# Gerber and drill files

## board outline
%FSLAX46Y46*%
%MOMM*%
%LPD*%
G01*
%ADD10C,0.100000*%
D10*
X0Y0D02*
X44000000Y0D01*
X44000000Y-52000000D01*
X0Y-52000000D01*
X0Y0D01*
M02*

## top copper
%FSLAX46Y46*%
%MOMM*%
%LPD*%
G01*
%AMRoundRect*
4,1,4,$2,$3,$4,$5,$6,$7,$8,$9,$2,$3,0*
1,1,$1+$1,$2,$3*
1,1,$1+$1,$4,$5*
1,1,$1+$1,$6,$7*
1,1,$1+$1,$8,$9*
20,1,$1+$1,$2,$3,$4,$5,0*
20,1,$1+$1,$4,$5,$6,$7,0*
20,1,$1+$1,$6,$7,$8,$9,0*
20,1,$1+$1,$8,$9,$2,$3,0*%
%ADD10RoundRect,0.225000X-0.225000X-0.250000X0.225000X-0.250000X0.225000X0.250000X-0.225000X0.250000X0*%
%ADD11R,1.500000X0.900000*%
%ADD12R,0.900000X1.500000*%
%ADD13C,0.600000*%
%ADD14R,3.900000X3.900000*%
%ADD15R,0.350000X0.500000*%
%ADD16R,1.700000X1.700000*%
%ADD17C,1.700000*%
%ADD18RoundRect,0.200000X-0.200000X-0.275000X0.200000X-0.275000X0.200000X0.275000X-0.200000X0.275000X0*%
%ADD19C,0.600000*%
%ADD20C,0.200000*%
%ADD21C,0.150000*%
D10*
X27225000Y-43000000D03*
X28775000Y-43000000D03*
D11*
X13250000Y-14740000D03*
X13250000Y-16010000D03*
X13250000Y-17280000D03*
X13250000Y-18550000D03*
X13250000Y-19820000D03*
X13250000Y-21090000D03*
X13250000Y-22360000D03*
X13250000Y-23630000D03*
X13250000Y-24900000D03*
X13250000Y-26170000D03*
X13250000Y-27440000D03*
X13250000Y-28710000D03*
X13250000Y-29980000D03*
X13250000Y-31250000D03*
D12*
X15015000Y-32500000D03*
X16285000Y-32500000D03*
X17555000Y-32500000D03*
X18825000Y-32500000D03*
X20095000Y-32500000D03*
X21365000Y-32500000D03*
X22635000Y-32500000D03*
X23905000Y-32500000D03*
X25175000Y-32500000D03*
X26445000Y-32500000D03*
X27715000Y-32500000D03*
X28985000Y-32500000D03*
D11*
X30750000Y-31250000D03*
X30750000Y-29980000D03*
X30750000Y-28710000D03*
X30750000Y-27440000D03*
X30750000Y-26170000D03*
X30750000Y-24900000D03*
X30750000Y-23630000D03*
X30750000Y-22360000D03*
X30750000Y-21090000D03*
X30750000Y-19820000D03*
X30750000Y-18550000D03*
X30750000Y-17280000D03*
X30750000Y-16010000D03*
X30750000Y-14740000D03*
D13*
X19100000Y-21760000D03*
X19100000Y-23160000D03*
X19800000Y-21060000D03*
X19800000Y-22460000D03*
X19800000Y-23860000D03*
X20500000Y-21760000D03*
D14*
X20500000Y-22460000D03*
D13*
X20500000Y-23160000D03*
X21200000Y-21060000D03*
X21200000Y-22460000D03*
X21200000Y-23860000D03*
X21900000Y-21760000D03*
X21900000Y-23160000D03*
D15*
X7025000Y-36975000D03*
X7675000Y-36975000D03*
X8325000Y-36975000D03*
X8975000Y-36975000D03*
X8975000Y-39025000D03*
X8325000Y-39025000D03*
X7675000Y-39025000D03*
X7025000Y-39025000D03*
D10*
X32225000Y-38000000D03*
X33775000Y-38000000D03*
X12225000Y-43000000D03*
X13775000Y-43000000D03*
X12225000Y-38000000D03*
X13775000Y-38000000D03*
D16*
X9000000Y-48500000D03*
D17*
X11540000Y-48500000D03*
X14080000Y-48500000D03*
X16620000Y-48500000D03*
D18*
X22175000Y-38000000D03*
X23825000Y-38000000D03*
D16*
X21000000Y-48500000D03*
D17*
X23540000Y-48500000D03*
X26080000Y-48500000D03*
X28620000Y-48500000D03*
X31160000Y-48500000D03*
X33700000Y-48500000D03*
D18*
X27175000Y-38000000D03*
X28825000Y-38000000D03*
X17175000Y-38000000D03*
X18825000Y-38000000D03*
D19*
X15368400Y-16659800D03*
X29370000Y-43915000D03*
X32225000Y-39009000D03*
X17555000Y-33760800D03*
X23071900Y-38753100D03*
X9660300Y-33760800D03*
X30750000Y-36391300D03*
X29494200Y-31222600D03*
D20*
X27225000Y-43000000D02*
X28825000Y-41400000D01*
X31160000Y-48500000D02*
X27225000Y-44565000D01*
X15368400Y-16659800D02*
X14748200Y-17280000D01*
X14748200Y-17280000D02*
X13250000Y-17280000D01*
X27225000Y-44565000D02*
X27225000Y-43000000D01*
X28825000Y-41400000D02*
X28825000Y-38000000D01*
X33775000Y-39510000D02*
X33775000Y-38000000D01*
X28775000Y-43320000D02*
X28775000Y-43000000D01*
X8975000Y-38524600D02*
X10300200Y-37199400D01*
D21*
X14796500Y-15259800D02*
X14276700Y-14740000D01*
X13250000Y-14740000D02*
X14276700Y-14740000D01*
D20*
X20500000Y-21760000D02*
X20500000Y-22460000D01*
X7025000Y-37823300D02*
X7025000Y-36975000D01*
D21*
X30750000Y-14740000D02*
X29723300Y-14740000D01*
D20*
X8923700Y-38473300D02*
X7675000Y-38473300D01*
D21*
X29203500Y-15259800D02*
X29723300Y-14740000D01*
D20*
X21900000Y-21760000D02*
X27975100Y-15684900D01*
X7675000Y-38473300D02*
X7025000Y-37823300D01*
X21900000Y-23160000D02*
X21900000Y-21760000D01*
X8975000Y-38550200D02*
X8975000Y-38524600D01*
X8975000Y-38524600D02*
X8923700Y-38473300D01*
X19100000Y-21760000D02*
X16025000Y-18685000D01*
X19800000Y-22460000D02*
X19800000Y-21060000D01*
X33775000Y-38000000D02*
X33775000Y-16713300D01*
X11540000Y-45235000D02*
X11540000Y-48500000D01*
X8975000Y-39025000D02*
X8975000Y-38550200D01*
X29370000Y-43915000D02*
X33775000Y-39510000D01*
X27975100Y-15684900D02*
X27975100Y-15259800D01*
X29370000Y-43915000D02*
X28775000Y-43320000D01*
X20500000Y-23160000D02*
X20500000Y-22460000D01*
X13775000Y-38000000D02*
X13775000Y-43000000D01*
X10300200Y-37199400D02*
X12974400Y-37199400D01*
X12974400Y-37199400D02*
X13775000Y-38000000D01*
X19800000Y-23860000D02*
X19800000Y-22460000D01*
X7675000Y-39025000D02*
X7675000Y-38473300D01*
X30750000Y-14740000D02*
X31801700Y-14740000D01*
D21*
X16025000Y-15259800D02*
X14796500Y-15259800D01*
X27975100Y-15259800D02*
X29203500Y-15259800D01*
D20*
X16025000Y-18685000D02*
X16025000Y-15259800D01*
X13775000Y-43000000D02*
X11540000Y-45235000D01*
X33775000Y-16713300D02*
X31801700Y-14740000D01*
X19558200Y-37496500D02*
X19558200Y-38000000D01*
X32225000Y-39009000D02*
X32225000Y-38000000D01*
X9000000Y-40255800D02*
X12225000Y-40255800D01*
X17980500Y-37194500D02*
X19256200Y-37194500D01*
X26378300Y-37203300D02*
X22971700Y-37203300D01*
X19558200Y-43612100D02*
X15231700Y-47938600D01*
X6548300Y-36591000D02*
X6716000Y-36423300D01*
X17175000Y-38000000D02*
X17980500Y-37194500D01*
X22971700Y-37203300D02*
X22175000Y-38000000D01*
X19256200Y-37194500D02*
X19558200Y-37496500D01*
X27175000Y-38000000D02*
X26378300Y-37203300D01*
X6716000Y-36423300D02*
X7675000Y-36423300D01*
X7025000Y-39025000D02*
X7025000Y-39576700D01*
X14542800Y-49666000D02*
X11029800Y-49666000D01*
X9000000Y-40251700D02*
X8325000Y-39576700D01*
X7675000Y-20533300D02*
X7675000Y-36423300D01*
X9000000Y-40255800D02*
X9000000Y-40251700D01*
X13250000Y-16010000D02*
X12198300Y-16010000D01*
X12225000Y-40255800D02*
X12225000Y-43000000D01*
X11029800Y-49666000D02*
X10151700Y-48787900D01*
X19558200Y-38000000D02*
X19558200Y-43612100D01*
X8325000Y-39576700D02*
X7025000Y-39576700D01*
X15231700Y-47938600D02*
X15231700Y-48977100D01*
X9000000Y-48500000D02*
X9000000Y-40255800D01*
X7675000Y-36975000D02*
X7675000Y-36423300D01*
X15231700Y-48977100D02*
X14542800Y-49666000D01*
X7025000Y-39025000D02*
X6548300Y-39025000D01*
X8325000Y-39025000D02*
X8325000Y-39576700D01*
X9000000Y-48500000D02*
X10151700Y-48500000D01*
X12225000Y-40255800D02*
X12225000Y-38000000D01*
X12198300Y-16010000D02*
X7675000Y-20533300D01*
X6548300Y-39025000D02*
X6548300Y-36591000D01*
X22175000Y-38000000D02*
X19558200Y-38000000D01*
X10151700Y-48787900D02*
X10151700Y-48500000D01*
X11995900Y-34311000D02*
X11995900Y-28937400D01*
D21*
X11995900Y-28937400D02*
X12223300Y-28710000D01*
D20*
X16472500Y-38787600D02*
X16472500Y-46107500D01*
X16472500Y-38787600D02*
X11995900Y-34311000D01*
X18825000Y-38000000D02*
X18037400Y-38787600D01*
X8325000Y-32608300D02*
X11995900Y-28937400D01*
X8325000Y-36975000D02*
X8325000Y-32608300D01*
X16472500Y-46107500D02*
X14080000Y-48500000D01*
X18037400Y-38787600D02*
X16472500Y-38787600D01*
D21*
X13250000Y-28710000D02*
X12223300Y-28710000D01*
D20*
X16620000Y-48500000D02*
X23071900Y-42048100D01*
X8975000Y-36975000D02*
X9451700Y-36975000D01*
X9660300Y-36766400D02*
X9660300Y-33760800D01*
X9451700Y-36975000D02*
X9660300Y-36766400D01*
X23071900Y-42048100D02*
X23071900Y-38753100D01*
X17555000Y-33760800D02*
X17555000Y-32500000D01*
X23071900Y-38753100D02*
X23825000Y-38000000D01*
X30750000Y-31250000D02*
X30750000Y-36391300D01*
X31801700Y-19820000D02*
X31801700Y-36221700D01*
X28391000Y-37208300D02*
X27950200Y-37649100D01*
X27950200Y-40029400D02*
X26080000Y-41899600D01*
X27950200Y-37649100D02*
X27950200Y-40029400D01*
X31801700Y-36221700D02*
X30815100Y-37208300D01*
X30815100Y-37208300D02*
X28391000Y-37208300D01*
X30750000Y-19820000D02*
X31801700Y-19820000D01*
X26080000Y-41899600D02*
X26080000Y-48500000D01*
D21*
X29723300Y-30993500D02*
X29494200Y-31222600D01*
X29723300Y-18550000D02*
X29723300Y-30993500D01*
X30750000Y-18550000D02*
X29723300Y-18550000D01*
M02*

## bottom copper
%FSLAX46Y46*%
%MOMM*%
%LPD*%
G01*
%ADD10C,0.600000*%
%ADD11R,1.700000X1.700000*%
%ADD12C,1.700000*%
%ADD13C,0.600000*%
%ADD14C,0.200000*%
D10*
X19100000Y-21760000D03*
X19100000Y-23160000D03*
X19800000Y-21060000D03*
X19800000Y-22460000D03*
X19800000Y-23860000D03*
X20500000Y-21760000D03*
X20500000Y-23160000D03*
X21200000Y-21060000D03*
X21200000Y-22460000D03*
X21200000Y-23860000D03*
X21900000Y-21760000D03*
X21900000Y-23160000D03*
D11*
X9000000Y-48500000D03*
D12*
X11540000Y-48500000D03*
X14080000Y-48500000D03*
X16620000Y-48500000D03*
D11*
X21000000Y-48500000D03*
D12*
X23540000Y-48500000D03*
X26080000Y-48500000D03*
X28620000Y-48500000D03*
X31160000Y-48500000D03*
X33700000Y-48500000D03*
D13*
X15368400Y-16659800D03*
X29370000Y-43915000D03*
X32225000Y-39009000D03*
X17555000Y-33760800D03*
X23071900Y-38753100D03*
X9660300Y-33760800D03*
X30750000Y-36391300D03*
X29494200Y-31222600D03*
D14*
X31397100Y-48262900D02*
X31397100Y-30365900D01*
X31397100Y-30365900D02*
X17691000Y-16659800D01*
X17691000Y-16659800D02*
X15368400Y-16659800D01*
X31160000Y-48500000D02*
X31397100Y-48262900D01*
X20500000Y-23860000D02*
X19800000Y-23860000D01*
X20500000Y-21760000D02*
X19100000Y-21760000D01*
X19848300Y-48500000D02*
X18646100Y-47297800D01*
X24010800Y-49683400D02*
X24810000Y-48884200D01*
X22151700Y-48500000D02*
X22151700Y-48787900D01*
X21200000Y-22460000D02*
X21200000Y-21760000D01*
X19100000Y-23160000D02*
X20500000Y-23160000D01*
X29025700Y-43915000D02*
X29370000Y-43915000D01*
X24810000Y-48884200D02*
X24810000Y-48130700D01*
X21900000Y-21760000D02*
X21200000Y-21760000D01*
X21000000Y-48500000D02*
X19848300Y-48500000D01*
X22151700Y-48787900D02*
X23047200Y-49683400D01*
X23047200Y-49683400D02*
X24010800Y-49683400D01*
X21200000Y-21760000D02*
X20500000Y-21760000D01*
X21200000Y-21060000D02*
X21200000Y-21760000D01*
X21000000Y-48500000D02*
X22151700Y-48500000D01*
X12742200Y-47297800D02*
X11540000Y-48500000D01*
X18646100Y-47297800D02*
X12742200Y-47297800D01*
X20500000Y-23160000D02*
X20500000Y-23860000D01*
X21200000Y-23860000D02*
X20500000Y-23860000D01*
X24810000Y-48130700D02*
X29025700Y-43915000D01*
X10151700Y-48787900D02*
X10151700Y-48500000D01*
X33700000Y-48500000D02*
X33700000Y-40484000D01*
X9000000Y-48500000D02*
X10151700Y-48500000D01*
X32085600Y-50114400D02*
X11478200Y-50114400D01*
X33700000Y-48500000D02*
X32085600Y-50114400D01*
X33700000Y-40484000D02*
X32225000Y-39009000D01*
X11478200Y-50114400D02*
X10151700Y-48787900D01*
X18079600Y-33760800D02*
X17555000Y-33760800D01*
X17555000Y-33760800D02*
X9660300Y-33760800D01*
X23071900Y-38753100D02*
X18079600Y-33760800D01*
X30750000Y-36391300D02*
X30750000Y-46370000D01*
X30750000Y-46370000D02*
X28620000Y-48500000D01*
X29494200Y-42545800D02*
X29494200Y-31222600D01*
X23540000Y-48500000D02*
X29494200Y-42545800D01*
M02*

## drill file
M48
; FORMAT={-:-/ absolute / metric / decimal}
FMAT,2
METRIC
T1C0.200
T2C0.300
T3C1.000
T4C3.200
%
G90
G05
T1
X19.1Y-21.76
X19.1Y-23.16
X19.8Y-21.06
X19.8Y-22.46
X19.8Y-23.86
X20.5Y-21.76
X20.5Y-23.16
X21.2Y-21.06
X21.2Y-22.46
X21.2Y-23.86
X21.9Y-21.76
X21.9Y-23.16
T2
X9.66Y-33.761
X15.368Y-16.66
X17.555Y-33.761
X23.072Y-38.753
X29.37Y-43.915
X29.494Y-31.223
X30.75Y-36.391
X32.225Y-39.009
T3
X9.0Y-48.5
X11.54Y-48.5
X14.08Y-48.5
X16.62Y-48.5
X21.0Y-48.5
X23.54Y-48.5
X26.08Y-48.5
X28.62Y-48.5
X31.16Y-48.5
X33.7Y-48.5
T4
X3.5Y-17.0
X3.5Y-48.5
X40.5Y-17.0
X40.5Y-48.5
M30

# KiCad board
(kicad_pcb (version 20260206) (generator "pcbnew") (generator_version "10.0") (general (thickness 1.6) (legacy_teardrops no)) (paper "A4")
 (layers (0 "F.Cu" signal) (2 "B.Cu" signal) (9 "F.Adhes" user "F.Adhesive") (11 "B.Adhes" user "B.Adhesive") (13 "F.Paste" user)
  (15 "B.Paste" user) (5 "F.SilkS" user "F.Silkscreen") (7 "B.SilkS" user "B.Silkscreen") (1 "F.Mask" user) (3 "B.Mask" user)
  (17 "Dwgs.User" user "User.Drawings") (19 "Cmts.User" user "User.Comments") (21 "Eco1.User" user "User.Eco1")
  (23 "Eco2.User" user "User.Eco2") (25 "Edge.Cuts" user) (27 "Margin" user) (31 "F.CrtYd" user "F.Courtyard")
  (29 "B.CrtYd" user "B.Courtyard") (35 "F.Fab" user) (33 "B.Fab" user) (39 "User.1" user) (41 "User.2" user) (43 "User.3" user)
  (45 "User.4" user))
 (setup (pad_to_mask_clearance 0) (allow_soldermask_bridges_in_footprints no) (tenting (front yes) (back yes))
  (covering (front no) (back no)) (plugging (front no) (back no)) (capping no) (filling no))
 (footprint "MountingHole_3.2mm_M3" (layer "F.Cu") (at 3.5 17)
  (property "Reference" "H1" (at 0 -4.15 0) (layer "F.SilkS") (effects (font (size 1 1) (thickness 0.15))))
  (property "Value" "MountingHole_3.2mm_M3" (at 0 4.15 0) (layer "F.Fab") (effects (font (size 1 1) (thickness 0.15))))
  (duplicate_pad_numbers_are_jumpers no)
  (pad "" np_thru_hole circle (at 0 0) (size 3.2 3.2) (drill 3.2) (layers "*.Cu" "*.Mask")))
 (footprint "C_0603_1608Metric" (layer "F.Cu") (at 28 43)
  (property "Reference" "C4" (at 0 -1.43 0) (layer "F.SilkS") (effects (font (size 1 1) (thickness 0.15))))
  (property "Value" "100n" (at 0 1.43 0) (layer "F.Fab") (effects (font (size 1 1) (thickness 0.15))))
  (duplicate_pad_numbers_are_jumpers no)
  (pad "1" smd roundrect (at -0.775 0) (size 0.9 0.95) (layers "F.Cu" "F.Mask" "F.Paste") (roundrect_rratio 0.25) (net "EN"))
  (pad "2" smd roundrect (at 0.775 0) (size 0.9 0.95) (layers "F.Cu" "F.Mask" "F.Paste") (roundrect_rratio 0.25) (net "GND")))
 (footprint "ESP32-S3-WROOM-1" (layer "F.Cu") (at 22 20)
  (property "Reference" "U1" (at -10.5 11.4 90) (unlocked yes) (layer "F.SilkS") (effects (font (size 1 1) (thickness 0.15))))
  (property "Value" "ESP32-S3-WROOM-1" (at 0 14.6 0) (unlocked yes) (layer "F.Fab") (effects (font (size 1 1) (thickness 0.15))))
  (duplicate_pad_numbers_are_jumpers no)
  (pad "" smd rect (at -2.9 1.06) (size 0.9 0.9) (layers "F.Paste"))
  (pad "" smd rect (at -2.9 2.46 270) (size 0.9 0.9) (layers "F.Paste"))
  (pad "" smd rect (at -2.9 3.86) (size 0.9 0.9) (layers "F.Paste"))
  (pad "" smd rect (at -1.5 1.06 270) (size 0.9 0.9) (layers "F.Paste"))
  (pad "" smd rect (at -1.5 2.46 270) (size 0.9 0.9) (layers "F.Paste"))
  (pad "" smd rect (at -1.5 3.86 270) (size 0.9 0.9) (layers "F.Paste"))
  (pad "" smd rect (at -0.1 1.06 270) (size 0.9 0.9) (layers "F.Paste"))
  (pad "" smd rect (at -0.1 2.46 270) (size 0.9 0.9) (layers "F.Paste"))
  (pad "" smd rect (at -0.1 3.86 270) (size 0.9 0.9) (layers "F.Paste"))
  (pad "1" smd rect (at -8.75 -5.26) (size 1.5 0.9) (layers "F.Cu" "F.Mask" "F.Paste") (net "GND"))
  (pad "2" smd rect (at -8.75 -3.99) (size 1.5 0.9) (layers "F.Cu" "F.Mask" "F.Paste") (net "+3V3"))
  (pad "3" smd rect (at -8.75 -2.72) (size 1.5 0.9) (layers "F.Cu" "F.Mask" "F.Paste") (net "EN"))
  (pad "4" smd rect (at -8.75 -1.45) (size 1.5 0.9) (layers "F.Cu" "F.Mask" "F.Paste") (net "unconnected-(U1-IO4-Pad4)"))
  (pad "5" smd rect (at -8.75 -0.18) (size 1.5 0.9) (layers "F.Cu" "F.Mask" "F.Paste") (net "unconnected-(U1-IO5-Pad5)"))
  (pad "6" smd rect (at -8.75 1.09) (size 1.5 0.9) (layers "F.Cu" "F.Mask" "F.Paste") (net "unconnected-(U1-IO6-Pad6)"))
  (pad "7" smd rect (at -8.75 2.36) (size 1.5 0.9) (layers "F.Cu" "F.Mask" "F.Paste") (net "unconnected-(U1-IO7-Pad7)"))
  (pad "8" smd rect (at -8.75 3.63) (size 1.5 0.9) (layers "F.Cu" "F.Mask" "F.Paste") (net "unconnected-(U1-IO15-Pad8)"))
  (pad "9" smd rect (at -8.75 4.9) (size 1.5 0.9) (layers "F.Cu" "F.Mask" "F.Paste") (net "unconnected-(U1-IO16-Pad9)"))
  (pad "10" smd rect (at -8.75 6.17) (size 1.5 0.9) (layers "F.Cu" "F.Mask" "F.Paste") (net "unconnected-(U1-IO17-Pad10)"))
  (pad "11" smd rect (at -8.75 7.44) (size 1.5 0.9) (layers "F.Cu" "F.Mask" "F.Paste") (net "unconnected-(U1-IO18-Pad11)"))
  (pad "12" smd rect (at -8.75 8.71) (size 1.5 0.9) (layers "F.Cu" "F.Mask" "F.Paste") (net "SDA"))
  (pad "13" smd rect (at -8.75 9.98) (size 1.5 0.9) (layers "F.Cu" "F.Mask" "F.Paste") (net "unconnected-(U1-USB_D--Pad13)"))
  (pad "14" smd rect (at -8.75 11.25 180) (size 1.5 0.9) (layers "F.Cu" "F.Mask" "F.Paste") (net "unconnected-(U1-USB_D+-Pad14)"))
  (pad "15" smd rect (at -6.985 12.5 270) (size 1.5 0.9) (layers "F.Cu" "F.Mask" "F.Paste") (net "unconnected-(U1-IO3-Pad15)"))
  (pad "16" smd rect (at -5.715 12.5 270) (size 1.5 0.9) (layers "F.Cu" "F.Mask" "F.Paste") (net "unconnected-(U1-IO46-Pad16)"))
  (pad "17" smd rect (at -4.445 12.5 270) (size 1.5 0.9) (layers "F.Cu" "F.Mask" "F.Paste") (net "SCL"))
  (pad "18" smd rect (at -3.175 12.5 270) (size 1.5 0.9) (layers "F.Cu" "F.Mask" "F.Paste") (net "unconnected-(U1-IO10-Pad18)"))
  (pad "19" smd rect (at -1.905 12.5 270) (size 1.5 0.9) (layers "F.Cu" "F.Mask" "F.Paste") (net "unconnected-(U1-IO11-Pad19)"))
  (pad "20" smd rect (at -0.635 12.5 270) (size 1.5 0.9) (layers "F.Cu" "F.Mask" "F.Paste") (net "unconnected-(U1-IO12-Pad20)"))
  (pad "21" smd rect (at 0.635 12.5 270) (size 1.5 0.9) (layers "F.Cu" "F.Mask" "F.Paste") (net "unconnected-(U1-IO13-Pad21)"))
  (pad "22" smd rect (at 1.905 12.5 270) (size 1.5 0.9) (layers "F.Cu" "F.Mask" "F.Paste") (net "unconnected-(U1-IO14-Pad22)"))
  (pad "23" smd rect (at 3.175 12.5 270) (size 1.5 0.9) (layers "F.Cu" "F.Mask" "F.Paste") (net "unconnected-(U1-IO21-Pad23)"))
  (pad "24" smd rect (at 4.445 12.5 270) (size 1.5 0.9) (layers "F.Cu" "F.Mask" "F.Paste") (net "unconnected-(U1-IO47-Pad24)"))
  (pad "25" smd rect (at 5.715 12.5 270) (size 1.5 0.9) (layers "F.Cu" "F.Mask" "F.Paste") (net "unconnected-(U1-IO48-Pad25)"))
  (pad "26" smd rect (at 6.985 12.5 270) (size 1.5 0.9) (layers "F.Cu" "F.Mask" "F.Paste") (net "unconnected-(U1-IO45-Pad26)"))
  (pad "27" smd rect (at 8.75 11.25) (size 1.5 0.9) (layers "F.Cu" "F.Mask" "F.Paste") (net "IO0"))
  (pad "28" smd rect (at 8.75 9.98) (size 1.5 0.9) (layers "F.Cu" "F.Mask" "F.Paste") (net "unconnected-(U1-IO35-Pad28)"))
  (pad "29" smd rect (at 8.75 8.71) (size 1.5 0.9) (layers "F.Cu" "F.Mask" "F.Paste") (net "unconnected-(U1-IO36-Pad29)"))
  (pad "30" smd rect (at 8.75 7.44) (size 1.5 0.9) (layers "F.Cu" "F.Mask" "F.Paste") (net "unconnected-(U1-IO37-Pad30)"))
  (pad "31" smd rect (at 8.75 6.17) (size 1.5 0.9) (layers "F.Cu" "F.Mask" "F.Paste") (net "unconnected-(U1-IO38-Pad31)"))
  (pad "32" smd rect (at 8.75 4.9) (size 1.5 0.9) (layers "F.Cu" "F.Mask" "F.Paste") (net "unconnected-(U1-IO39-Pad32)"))
  (pad "33" smd rect (at 8.75 3.63) (size 1.5 0.9) (layers "F.Cu" "F.Mask" "F.Paste") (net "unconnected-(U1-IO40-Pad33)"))
  (pad "34" smd rect (at 8.75 2.36) (size 1.5 0.9) (layers "F.Cu" "F.Mask" "F.Paste") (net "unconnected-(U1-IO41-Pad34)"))
  (pad "35" smd rect (at 8.75 1.09) (size 1.5 0.9) (layers "F.Cu" "F.Mask" "F.Paste") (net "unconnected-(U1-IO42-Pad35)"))
  (pad "36" smd rect (at 8.75 -0.18) (size 1.5 0.9) (layers "F.Cu" "F.Mask" "F.Paste") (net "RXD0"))
  (pad "37" smd rect (at 8.75 -1.45) (size 1.5 0.9) (layers "F.Cu" "F.Mask" "F.Paste") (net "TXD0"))
  (pad "38" smd rect (at 8.75 -2.72) (size 1.5 0.9) (layers "F.Cu" "F.Mask" "F.Paste") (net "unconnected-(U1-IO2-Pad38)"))
  (pad "39" smd rect (at 8.75 -3.99) (size 1.5 0.9) (layers "F.Cu" "F.Mask" "F.Paste") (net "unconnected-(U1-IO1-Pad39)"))
  (pad "40" smd rect (at 8.75 -5.26) (size 1.5 0.9) (layers "F.Cu" "F.Mask" "F.Paste") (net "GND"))
  (pad "41" thru_hole circle (at -2.9 1.76 90) (size 0.6 0.6) (drill 0.2) (layers "*.Cu" "F.Mask") (remove_unused_layers no) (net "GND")
   (zone_connect 2))
  (pad "41" thru_hole circle (at -2.9 3.16) (size 0.6 0.6) (drill 0.2) (layers "*.Cu" "F.Mask") (remove_unused_layers no) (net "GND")
   (zone_connect 2))
  (pad "41" thru_hole circle (at -2.2 1.06) (size 0.6 0.6) (drill 0.2) (layers "*.Cu" "F.Mask") (remove_unused_layers no) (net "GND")
   (zone_connect 2))
  (pad "41" thru_hole circle (at -2.2 2.46) (size 0.6 0.6) (drill 0.2) (layers "*.Cu" "F.Mask") (remove_unused_layers no) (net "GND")
   (zone_connect 2))
  (pad "41" thru_hole circle (at -2.2 3.86) (size 0.6 0.6) (drill 0.2) (layers "*.Cu" "F.Mask") (remove_unused_layers no) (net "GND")
   (zone_connect 2))
  (pad "41" thru_hole circle (at -1.5 1.76) (size 0.6 0.6) (drill 0.2) (layers "*.Cu" "F.Mask") (remove_unused_layers no) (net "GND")
   (zone_connect 2))
  (pad "41" smd rect (at -1.5 2.46 270) (size 3.9 3.9) (layers "F.Cu" "F.Mask") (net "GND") (zone_connect 2))
  (pad "41" thru_hole circle (at -1.5 3.16) (size 0.6 0.6) (drill 0.2) (layers "*.Cu" "F.Mask") (remove_unused_layers no) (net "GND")
   (zone_connect 2))
  (pad "41" thru_hole circle (at -0.8 1.06) (size 0.6 0.6) (drill 0.2) (layers "*.Cu" "F.Mask") (remove_unused_layers no) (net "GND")
   (zone_connect 2))
  (pad "41" thru_hole circle (at -0.8 2.46) (size 0.6 0.6) (drill 0.2) (layers "*.Cu" "F.Mask") (remove_unused_layers no) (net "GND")
   (zone_connect 2))
  (pad "41" thru_hole circle (at -0.8 3.86) (size 0.6 0.6) (drill 0.2) (layers "*.Cu" "F.Mask") (remove_unused_layers no) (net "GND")
   (zone_connect 2))
  (pad "41" thru_hole circle (at -0.1 1.76) (size 0.6 0.6) (drill 0.2) (layers "*.Cu" "F.Mask") (remove_unused_layers no) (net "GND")
   (zone_connect 2))
  (pad "41" thru_hole circle (at -0.1 3.16) (size 0.6 0.6) (drill 0.2) (layers "*.Cu" "F.Mask") (remove_unused_layers no) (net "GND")
   (zone_connect 2))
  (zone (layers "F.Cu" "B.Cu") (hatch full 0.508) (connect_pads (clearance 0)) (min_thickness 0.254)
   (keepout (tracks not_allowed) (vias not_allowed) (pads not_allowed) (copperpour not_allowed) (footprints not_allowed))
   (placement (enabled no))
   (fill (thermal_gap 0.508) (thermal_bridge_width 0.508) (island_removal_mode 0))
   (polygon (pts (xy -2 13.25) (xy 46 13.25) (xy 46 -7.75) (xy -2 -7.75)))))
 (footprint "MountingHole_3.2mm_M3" (layer "F.Cu") (at 40.5 48.5)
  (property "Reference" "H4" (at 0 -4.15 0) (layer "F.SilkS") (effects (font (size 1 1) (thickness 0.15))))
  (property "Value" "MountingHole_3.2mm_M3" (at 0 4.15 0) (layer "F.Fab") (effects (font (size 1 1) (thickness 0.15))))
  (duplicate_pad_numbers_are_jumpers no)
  (pad "" np_thru_hole circle (at 0 0) (size 3.2 3.2) (drill 3.2) (layers "*.Cu" "*.Mask")))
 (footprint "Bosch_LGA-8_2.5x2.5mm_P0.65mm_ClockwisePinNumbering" (layer "F.Cu") (at 8 38)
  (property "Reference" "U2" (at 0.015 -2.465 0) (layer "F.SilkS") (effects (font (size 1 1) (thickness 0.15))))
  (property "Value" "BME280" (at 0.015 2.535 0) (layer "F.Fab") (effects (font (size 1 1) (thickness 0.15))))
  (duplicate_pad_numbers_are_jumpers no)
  (pad "1" smd rect (at -0.975 -1.025 90) (size 0.5 0.35) (layers "F.Cu" "F.Mask" "F.Paste") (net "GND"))
  (pad "2" smd rect (at -0.325 -1.025 90) (size 0.5 0.35) (layers "F.Cu" "F.Mask" "F.Paste") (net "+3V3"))
  (pad "3" smd rect (at 0.325 -1.025 90) (size 0.5 0.35) (layers "F.Cu" "F.Mask" "F.Paste") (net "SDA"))
  (pad "4" smd rect (at 0.975 -1.025 90) (size 0.5 0.35) (layers "F.Cu" "F.Mask" "F.Paste") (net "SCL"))
  (pad "5" smd rect (at 0.975 1.025 90) (size 0.5 0.35) (layers "F.Cu" "F.Mask" "F.Paste") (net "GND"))
  (pad "6" smd rect (at 0.325 1.025 90) (size 0.5 0.35) (layers "F.Cu" "F.Mask" "F.Paste") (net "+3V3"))
  (pad "7" smd rect (at -0.325 1.025 90) (size 0.5 0.35) (layers "F.Cu" "F.Mask" "F.Paste") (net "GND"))
  (pad "8" smd rect (at -0.975 1.025 90) (size 0.5 0.35) (layers "F.Cu" "F.Mask" "F.Paste") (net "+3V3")))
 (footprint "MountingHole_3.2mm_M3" (layer "F.Cu") (at 3.5 48.5)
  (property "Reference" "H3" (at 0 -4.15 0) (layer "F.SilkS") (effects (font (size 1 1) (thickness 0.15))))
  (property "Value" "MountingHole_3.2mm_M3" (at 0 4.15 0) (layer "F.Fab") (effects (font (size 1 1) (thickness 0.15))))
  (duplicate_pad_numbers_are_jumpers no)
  (pad "" np_thru_hole circle (at 0 0) (size 3.2 3.2) (drill 3.2) (layers "*.Cu" "*.Mask")))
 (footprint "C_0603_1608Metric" (layer "F.Cu") (at 33 38)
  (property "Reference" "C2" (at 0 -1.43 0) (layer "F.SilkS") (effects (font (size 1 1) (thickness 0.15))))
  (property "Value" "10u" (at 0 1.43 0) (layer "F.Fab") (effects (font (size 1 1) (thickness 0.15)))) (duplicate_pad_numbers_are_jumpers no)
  (pad "1" smd roundrect (at -0.775 0) (size 0.9 0.95) (layers "F.Cu" "F.Mask" "F.Paste") (roundrect_rratio 0.25) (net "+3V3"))
  (pad "2" smd roundrect (at 0.775 0) (size 0.9 0.95) (layers "F.Cu" "F.Mask" "F.Paste") (roundrect_rratio 0.25) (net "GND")))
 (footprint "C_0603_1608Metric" (layer "F.Cu") (at 13 43)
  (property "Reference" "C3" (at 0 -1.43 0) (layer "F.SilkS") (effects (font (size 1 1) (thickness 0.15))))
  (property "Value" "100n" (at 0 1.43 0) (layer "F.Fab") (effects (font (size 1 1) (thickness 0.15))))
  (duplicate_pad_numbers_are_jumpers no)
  (pad "1" smd roundrect (at -0.775 0) (size 0.9 0.95) (layers "F.Cu" "F.Mask" "F.Paste") (roundrect_rratio 0.25) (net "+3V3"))
  (pad "2" smd roundrect (at 0.775 0) (size 0.9 0.95) (layers "F.Cu" "F.Mask" "F.Paste") (roundrect_rratio 0.25) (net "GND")))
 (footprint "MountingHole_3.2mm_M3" (layer "F.Cu") (at 40.5 17)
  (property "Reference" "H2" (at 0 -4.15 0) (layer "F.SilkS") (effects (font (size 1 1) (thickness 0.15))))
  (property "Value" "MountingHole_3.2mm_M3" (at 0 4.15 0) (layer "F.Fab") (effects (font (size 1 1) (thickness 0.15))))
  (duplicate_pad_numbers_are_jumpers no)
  (pad "" np_thru_hole circle (at 0 0) (size 3.2 3.2) (drill 3.2) (layers "*.Cu" "*.Mask")))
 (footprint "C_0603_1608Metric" (layer "F.Cu") (at 13 38)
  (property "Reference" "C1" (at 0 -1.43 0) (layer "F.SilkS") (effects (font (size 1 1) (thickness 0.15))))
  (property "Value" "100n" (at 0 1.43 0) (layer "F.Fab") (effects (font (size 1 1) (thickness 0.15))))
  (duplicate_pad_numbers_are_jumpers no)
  (pad "1" smd roundrect (at -0.775 0) (size 0.9 0.95) (layers "F.Cu" "F.Mask" "F.Paste") (roundrect_rratio 0.25) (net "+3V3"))
  (pad "2" smd roundrect (at 0.775 0) (size 0.9 0.95) (layers "F.Cu" "F.Mask" "F.Paste") (roundrect_rratio 0.25) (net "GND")))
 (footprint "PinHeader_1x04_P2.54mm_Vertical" (layer "F.Cu") (at 9 48.5 90)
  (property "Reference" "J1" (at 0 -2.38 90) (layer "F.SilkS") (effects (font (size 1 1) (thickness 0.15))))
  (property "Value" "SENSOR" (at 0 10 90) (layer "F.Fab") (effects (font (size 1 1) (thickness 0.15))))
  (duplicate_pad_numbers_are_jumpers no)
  (pad "1" thru_hole rect (at 0 0 90) (size 1.7 1.7) (drill 1) (layers "*.Cu" "*.Mask") (remove_unused_layers no) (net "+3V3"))
  (pad "2" thru_hole circle (at 0 2.54 90) (size 1.7 1.7) (drill 1) (layers "*.Cu" "*.Mask") (remove_unused_layers no) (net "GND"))
  (pad "3" thru_hole circle (at 0 5.08 90) (size 1.7 1.7) (drill 1) (layers "*.Cu" "*.Mask") (remove_unused_layers no) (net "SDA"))
  (pad "4" thru_hole circle (at 0 7.62 90) (size 1.7 1.7) (drill 1) (layers "*.Cu" "*.Mask") (remove_unused_layers no) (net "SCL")))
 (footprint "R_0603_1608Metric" (layer "F.Cu") (at 23 38)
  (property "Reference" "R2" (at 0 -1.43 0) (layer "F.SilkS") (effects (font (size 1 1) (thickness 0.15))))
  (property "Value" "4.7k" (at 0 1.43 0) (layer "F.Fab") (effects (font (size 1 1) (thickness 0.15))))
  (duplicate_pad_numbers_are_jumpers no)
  (pad "1" smd roundrect (at -0.825 0) (size 0.8 0.95) (layers "F.Cu" "F.Mask" "F.Paste") (roundrect_rratio 0.25) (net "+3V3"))
  (pad "2" smd roundrect (at 0.825 0) (size 0.8 0.95) (layers "F.Cu" "F.Mask" "F.Paste") (roundrect_rratio 0.25) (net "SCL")))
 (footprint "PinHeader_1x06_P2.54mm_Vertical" (layer "F.Cu") (at 21 48.5 90)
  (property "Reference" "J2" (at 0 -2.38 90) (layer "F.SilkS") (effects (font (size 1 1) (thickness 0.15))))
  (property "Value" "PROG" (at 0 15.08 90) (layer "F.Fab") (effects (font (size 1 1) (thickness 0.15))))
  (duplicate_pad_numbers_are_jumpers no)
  (pad "1" thru_hole rect (at 0 0 90) (size 1.7 1.7) (drill 1) (layers "*.Cu" "*.Mask") (remove_unused_layers no) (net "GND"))
  (pad "2" thru_hole circle (at 0 2.54 90) (size 1.7 1.7) (drill 1) (layers "*.Cu" "*.Mask") (remove_unused_layers no) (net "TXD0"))
  (pad "3" thru_hole circle (at 0 5.08 90) (size 1.7 1.7) (drill 1) (layers "*.Cu" "*.Mask") (remove_unused_layers no) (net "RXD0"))
  (pad "4" thru_hole circle (at 0 7.62 90) (size 1.7 1.7) (drill 1) (layers "*.Cu" "*.Mask") (remove_unused_layers no) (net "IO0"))
  (pad "5" thru_hole circle (at 0 10.16 90) (size 1.7 1.7) (drill 1) (layers "*.Cu" "*.Mask") (remove_unused_layers no) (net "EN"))
  (pad "6" thru_hole circle (at 0 12.7 90) (size 1.7 1.7) (drill 1) (layers "*.Cu" "*.Mask") (remove_unused_layers no) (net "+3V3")))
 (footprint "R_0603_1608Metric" (layer "F.Cu") (at 28 38)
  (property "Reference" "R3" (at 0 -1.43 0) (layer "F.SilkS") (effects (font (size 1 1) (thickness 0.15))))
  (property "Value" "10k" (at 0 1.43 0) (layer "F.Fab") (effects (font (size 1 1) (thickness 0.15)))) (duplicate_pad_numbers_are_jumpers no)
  (pad "1" smd roundrect (at -0.825 0) (size 0.8 0.95) (layers "F.Cu" "F.Mask" "F.Paste") (roundrect_rratio 0.25) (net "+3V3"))
  (pad "2" smd roundrect (at 0.825 0) (size 0.8 0.95) (layers "F.Cu" "F.Mask" "F.Paste") (roundrect_rratio 0.25) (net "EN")))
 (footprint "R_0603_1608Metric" (layer "F.Cu") (at 18 38)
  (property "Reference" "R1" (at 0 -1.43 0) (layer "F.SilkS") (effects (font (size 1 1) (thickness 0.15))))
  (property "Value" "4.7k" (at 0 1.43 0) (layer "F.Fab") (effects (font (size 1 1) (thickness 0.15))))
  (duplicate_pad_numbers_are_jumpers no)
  (pad "1" smd roundrect (at -0.825 0) (size 0.8 0.95) (layers "F.Cu" "F.Mask" "F.Paste") (roundrect_rratio 0.25) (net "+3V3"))
  (pad "2" smd roundrect (at 0.825 0) (size 0.8 0.95) (layers "F.Cu" "F.Mask" "F.Paste") (roundrect_rratio 0.25) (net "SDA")))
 (gr_rect (start 0 0) (end 44 52) (stroke (width 0.1) (type default)) (fill no) (layer "Edge.Cuts"))
 (segment (start 27.225 43) (end 28.825 41.4) (width 0.2) (layer "F.Cu") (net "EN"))
 (segment (start 31.16 48.5) (end 27.225 44.565) (width 0.2) (layer "F.Cu") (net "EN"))
 (segment (start 15.3684 16.6598) (end 14.7482 17.28) (width 0.2) (layer "F.Cu") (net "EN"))
 (segment (start 14.7482 17.28) (end 13.25 17.28) (width 0.2) (layer "F.Cu") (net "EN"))
 (segment (start 27.225 44.565) (end 27.225 43) (width 0.2) (layer "F.Cu") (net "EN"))
 (segment (start 28.825 41.4) (end 28.825 38) (width 0.2) (layer "F.Cu") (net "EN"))
 (via (at 15.3684 16.6598) (size 0.6) (drill 0.3) (layers "F.Cu" "B.Cu") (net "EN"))
 (segment (start 31.3971 48.2629) (end 31.3971 30.3659) (width 0.2) (layer "B.Cu") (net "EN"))
 (segment (start 31.3971 30.3659) (end 17.691 16.6598) (width 0.2) (layer "B.Cu") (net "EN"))
 (segment (start 17.691 16.6598) (end 15.3684 16.6598) (width 0.2) (layer "B.Cu") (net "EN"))
 (segment (start 31.16 48.5) (end 31.3971 48.2629) (width 0.2) (layer "B.Cu") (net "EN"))
 (segment (start 33.775 39.51) (end 33.775 38) (width 0.2) (layer "F.Cu") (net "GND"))
 (segment (start 28.775 43.32) (end 28.775 43) (width 0.2) (layer "F.Cu") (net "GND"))
 (segment (start 8.975 38.5246) (end 10.3002 37.1994) (width 0.2) (layer "F.Cu") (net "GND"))
 (segment (start 14.7965 15.2598) (end 14.2767 14.74) (width 0.15) (layer "F.Cu") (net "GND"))
 (segment (start 13.25 14.74) (end 14.2767 14.74) (width 0.15) (layer "F.Cu") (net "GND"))
 (segment (start 20.5 21.76) (end 20.5 22.46) (width 0.2) (layer "F.Cu") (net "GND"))
 (segment (start 7.025 37.8233) (end 7.025 36.975) (width 0.2) (layer "F.Cu") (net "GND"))
 (segment (start 30.75 14.74) (end 29.7233 14.74) (width 0.15) (layer "F.Cu") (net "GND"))
 (segment (start 8.9237 38.4733) (end 7.675 38.4733) (width 0.2) (layer "F.Cu") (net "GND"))
 (segment (start 29.2035 15.2598) (end 29.7233 14.74) (width 0.15) (layer "F.Cu") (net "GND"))
 (segment (start 21.9 21.76) (end 27.9751 15.6849) (width 0.2) (layer "F.Cu") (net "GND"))
 (segment (start 7.675 38.4733) (end 7.025 37.8233) (width 0.2) (layer "F.Cu") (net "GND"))
 (segment (start 21.9 23.16) (end 21.9 21.76) (width 0.2) (layer "F.Cu") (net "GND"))
 (segment (start 8.975 38.5502) (end 8.975 38.5246) (width 0.2) (layer "F.Cu") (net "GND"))
 (segment (start 8.975 38.5246) (end 8.9237 38.4733) (width 0.2) (layer "F.Cu") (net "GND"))
 (segment (start 19.1 21.76) (end 16.025 18.685) (width 0.2) (layer "F.Cu") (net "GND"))
 (segment (start 19.8 22.46) (end 19.8 21.06) (width 0.2) (layer "F.Cu") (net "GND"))
 (segment (start 33.775 38) (end 33.775 16.7133) (width 0.2) (layer "F.Cu") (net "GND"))
 (segment (start 11.54 45.235) (end 11.54 48.5) (width 0.2) (layer "F.Cu") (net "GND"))
 (segment (start 8.975 39.025) (end 8.975 38.5502) (width 0.2) (layer "F.Cu") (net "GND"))
 (segment (start 29.37 43.915) (end 33.775 39.51) (width 0.2) (layer "F.Cu") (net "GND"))
 (segment (start 27.9751 15.6849) (end 27.9751 15.2598) (width 0.2) (layer "F.Cu") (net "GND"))
 (segment (start 29.37 43.915) (end 28.775 43.32) (width 0.2) (layer "F.Cu") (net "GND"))
 (segment (start 20.5 23.16) (end 20.5 22.46) (width 0.2) (layer "F.Cu") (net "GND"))
 (segment (start 13.775 38) (end 13.775 43) (width 0.2) (layer "F.Cu") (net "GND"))
 (segment (start 10.3002 37.1994) (end 12.9744 37.1994) (width 0.2) (layer "F.Cu") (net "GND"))
 (segment (start 12.9744 37.1994) (end 13.775 38) (width 0.2) (layer "F.Cu") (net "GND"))
 (segment (start 19.8 23.86) (end 19.8 22.46) (width 0.2) (layer "F.Cu") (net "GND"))
 (segment (start 7.675 39.025) (end 7.675 38.4733) (width 0.2) (layer "F.Cu") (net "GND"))
 (segment (start 30.75 14.74) (end 31.8017 14.74) (width 0.2) (layer "F.Cu") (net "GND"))
 (segment (start 16.025 15.2598) (end 14.7965 15.2598) (width 0.15) (layer "F.Cu") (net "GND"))
 (segment (start 27.9751 15.2598) (end 29.2035 15.2598) (width 0.15) (layer "F.Cu") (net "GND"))
 (segment (start 16.025 18.685) (end 16.025 15.2598) (width 0.2) (layer "F.Cu") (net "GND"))
 (segment (start 13.775 43) (end 11.54 45.235) (width 0.2) (layer "F.Cu") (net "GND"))
 (segment (start 33.775 16.7133) (end 31.8017 14.74) (width 0.2) (layer "F.Cu") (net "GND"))
 (via (at 29.37 43.915) (size 0.6) (drill 0.3) (layers "F.Cu" "B.Cu") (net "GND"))
 (segment (start 20.5 23.86) (end 19.8 23.86) (width 0.2) (layer "B.Cu") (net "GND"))
 (segment (start 20.5 21.76) (end 19.1 21.76) (width 0.2) (layer "B.Cu") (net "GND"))
 (segment (start 19.8483 48.5) (end 18.6461 47.2978) (width 0.2) (layer "B.Cu") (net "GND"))
 (segment (start 24.0108 49.6834) (end 24.81 48.8842) (width 0.2) (layer "B.Cu") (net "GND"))
 (segment (start 22.1517 48.5) (end 22.1517 48.7879) (width 0.2) (layer "B.Cu") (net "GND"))
 (segment (start 21.2 22.46) (end 21.2 21.76) (width 0.2) (layer "B.Cu") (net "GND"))
 (segment (start 19.1 23.16) (end 20.5 23.16) (width 0.2) (layer "B.Cu") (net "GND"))
 (segment (start 29.0257 43.915) (end 29.37 43.915) (width 0.2) (layer "B.Cu") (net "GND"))
 (segment (start 24.81 48.8842) (end 24.81 48.1307) (width 0.2) (layer "B.Cu") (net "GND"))
 (segment (start 21.9 21.76) (end 21.2 21.76) (width 0.2) (layer "B.Cu") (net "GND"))
 (segment (start 21 48.5) (end 19.8483 48.5) (width 0.2) (layer "B.Cu") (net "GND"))
 (segment (start 22.1517 48.7879) (end 23.0472 49.6834) (width 0.2) (layer "B.Cu") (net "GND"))
 (segment (start 23.0472 49.6834) (end 24.0108 49.6834) (width 0.2) (layer "B.Cu") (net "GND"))
 (segment (start 21.2 21.76) (end 20.5 21.76) (width 0.2) (layer "B.Cu") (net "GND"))
 (segment (start 21.2 21.06) (end 21.2 21.76) (width 0.2) (layer "B.Cu") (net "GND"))
 (segment (start 21 48.5) (end 22.1517 48.5) (width 0.2) (layer "B.Cu") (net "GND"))
 (segment (start 12.7422 47.2978) (end 11.54 48.5) (width 0.2) (layer "B.Cu") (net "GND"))
 (segment (start 18.6461 47.2978) (end 12.7422 47.2978) (width 0.2) (layer "B.Cu") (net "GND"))
 (segment (start 20.5 23.16) (end 20.5 23.86) (width 0.2) (layer "B.Cu") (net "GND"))
 (segment (start 21.2 23.86) (end 20.5 23.86) (width 0.2) (layer "B.Cu") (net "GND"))
 (segment (start 24.81 48.1307) (end 29.0257 43.915) (width 0.2) (layer "B.Cu") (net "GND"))
 (segment (start 19.5582 37.4965) (end 19.5582 38) (width 0.2) (layer "F.Cu") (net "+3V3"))
 (segment (start 32.225 39.009) (end 32.225 38) (width 0.2) (layer "F.Cu") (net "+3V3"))
 (segment (start 9 40.2558) (end 12.225 40.2558) (width 0.2) (layer "F.Cu") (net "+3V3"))
 (segment (start 17.9805 37.1945) (end 19.2562 37.1945) (width 0.2) (layer "F.Cu") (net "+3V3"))
 (segment (start 26.3783 37.2033) (end 22.9717 37.2033) (width 0.2) (layer "F.Cu") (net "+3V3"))
 (segment (start 19.5582 43.6121) (end 15.2317 47.9386) (width 0.2) (layer "F.Cu") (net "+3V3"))
 (segment (start 6.5483 36.591) (end 6.716 36.4233) (width 0.2) (layer "F.Cu") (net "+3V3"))
 (segment (start 17.175 38) (end 17.9805 37.1945) (width 0.2) (layer "F.Cu") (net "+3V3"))
 (segment (start 22.9717 37.2033) (end 22.175 38) (width 0.2) (layer "F.Cu") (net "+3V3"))
 (segment (start 19.2562 37.1945) (end 19.5582 37.4965) (width 0.2) (layer "F.Cu") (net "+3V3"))
 (segment (start 27.175 38) (end 26.3783 37.2033) (width 0.2) (layer "F.Cu") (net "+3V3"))
 (segment (start 6.716 36.4233) (end 7.675 36.4233) (width 0.2) (layer "F.Cu") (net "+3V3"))
 (segment (start 7.025 39.025) (end 7.025 39.5767) (width 0.2) (layer "F.Cu") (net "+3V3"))
 (segment (start 14.5428 49.666) (end 11.0298 49.666) (width 0.2) (layer "F.Cu") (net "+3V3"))
 (segment (start 9 40.2517) (end 8.325 39.5767) (width 0.2) (layer "F.Cu") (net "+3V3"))
 (segment (start 7.675 20.5333) (end 7.675 36.4233) (width 0.2) (layer "F.Cu") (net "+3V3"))
 (segment (start 9 40.2558) (end 9 40.2517) (width 0.2) (layer "F.Cu") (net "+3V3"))
 (segment (start 13.25 16.01) (end 12.1983 16.01) (width 0.2) (layer "F.Cu") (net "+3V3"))
 (segment (start 12.225 40.2558) (end 12.225 43) (width 0.2) (layer "F.Cu") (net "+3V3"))
 (segment (start 11.0298 49.666) (end 10.1517 48.7879) (width 0.2) (layer "F.Cu") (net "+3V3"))
 (segment (start 19.5582 38) (end 19.5582 43.6121) (width 0.2) (layer "F.Cu") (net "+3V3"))
 (segment (start 8.325 39.5767) (end 7.025 39.5767) (width 0.2) (layer "F.Cu") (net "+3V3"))
 (segment (start 15.2317 47.9386) (end 15.2317 48.9771) (width 0.2) (layer "F.Cu") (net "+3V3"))
 (segment (start 9 48.5) (end 9 40.2558) (width 0.2) (layer "F.Cu") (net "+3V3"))
 (segment (start 7.675 36.975) (end 7.675 36.4233) (width 0.2) (layer "F.Cu") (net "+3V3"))
 (segment (start 15.2317 48.9771) (end 14.5428 49.666) (width 0.2) (layer "F.Cu") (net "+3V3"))
 (segment (start 7.025 39.025) (end 6.5483 39.025) (width 0.2) (layer "F.Cu") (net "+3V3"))
 (segment (start 8.325 39.025) (end 8.325 39.5767) (width 0.2) (layer "F.Cu") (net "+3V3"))
 (segment (start 9 48.5) (end 10.1517 48.5) (width 0.2) (layer "F.Cu") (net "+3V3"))
 (segment (start 12.225 40.2558) (end 12.225 38) (width 0.2) (layer "F.Cu") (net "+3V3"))
 (segment (start 12.1983 16.01) (end 7.675 20.5333) (width 0.2) (layer "F.Cu") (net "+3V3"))
 (segment (start 6.5483 39.025) (end 6.5483 36.591) (width 0.2) (layer "F.Cu") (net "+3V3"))
 (segment (start 22.175 38) (end 19.5582 38) (width 0.2) (layer "F.Cu") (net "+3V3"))
 (segment (start 10.1517 48.7879) (end 10.1517 48.5) (width 0.2) (layer "F.Cu") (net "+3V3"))
 (via (at 32.225 39.009) (size 0.6) (drill 0.3) (layers "F.Cu" "B.Cu") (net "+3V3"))
 (segment (start 10.1517 48.7879) (end 10.1517 48.5) (width 0.2) (layer "B.Cu") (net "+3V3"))
 (segment (start 33.7 48.5) (end 33.7 40.484) (width 0.2) (layer "B.Cu") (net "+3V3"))
 (segment (start 9 48.5) (end 10.1517 48.5) (width 0.2) (layer "B.Cu") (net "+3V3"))
 (segment (start 32.0856 50.1144) (end 11.4782 50.1144) (width 0.2) (layer "B.Cu") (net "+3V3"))
 (segment (start 33.7 48.5) (end 32.0856 50.1144) (width 0.2) (layer "B.Cu") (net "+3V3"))
 (segment (start 33.7 40.484) (end 32.225 39.009) (width 0.2) (layer "B.Cu") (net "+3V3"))
 (segment (start 11.4782 50.1144) (end 10.1517 48.7879) (width 0.2) (layer "B.Cu") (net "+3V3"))
 (segment (start 11.9959 34.311) (end 11.9959 28.9374) (width 0.2) (layer "F.Cu") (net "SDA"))
 (segment (start 11.9959 28.9374) (end 12.2233 28.71) (width 0.15) (layer "F.Cu") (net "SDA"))
 (segment (start 16.4725 38.7876) (end 16.4725 46.1075) (width 0.2) (layer "F.Cu") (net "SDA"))
 (segment (start 16.4725 38.7876) (end 11.9959 34.311) (width 0.2) (layer "F.Cu") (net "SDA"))
 (segment (start 18.825 38) (end 18.0374 38.7876) (width 0.2) (layer "F.Cu") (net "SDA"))
 (segment (start 8.325 32.6083) (end 11.9959 28.9374) (width 0.2) (layer "F.Cu") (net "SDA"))
 (segment (start 8.325 36.975) (end 8.325 32.6083) (width 0.2) (layer "F.Cu") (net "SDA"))
 (segment (start 16.4725 46.1075) (end 14.08 48.5) (width 0.2) (layer "F.Cu") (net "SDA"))
 (segment (start 18.0374 38.7876) (end 16.4725 38.7876) (width 0.2) (layer "F.Cu") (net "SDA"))
 (segment (start 13.25 28.71) (end 12.2233 28.71) (width 0.15) (layer "F.Cu") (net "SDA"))
 (segment (start 16.62 48.5) (end 23.0719 42.0481) (width 0.2) (layer "F.Cu") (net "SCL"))
 (segment (start 8.975 36.975) (end 9.4517 36.975) (width 0.2) (layer "F.Cu") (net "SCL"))
 (segment (start 9.6603 36.7664) (end 9.6603 33.7608) (width 0.2) (layer "F.Cu") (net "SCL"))
 (segment (start 9.4517 36.975) (end 9.6603 36.7664) (width 0.2) (layer "F.Cu") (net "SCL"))
 (segment (start 23.0719 42.0481) (end 23.0719 38.7531) (width 0.2) (layer "F.Cu") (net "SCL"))
 (segment (start 17.555 33.7608) (end 17.555 32.5) (width 0.2) (layer "F.Cu") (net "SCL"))
 (segment (start 23.0719 38.7531) (end 23.825 38) (width 0.2) (layer "F.Cu") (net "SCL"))
 (via (at 17.555 33.7608) (size 0.6) (drill 0.3) (layers "F.Cu" "B.Cu") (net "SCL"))
 (via (at 23.0719 38.7531) (size 0.6) (drill 0.3) (layers "F.Cu" "B.Cu") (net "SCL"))
 (via (at 9.6603 33.7608) (size 0.6) (drill 0.3) (layers "F.Cu" "B.Cu") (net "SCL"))
 (segment (start 18.0796 33.7608) (end 17.555 33.7608) (width 0.2) (layer "B.Cu") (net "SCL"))
 (segment (start 17.555 33.7608) (end 9.6603 33.7608) (width 0.2) (layer "B.Cu") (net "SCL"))
 (segment (start 23.0719 38.7531) (end 18.0796 33.7608) (width 0.2) (layer "B.Cu") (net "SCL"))
 (segment (start 30.75 31.25) (end 30.75 36.3913) (width 0.2) (layer "F.Cu") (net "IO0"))
 (via (at 30.75 36.3913) (size 0.6) (drill 0.3) (layers "F.Cu" "B.Cu") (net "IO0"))
 (segment (start 30.75 36.3913) (end 30.75 46.37) (width 0.2) (layer "B.Cu") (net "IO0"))
 (segment (start 30.75 46.37) (end 28.62 48.5) (width 0.2) (layer "B.Cu") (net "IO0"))
 (segment (start 31.8017 19.82) (end 31.8017 36.2217) (width 0.2) (layer "F.Cu") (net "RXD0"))
 (segment (start 28.391 37.2083) (end 27.9502 37.6491) (width 0.2) (layer "F.Cu") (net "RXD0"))
 (segment (start 27.9502 40.0294) (end 26.08 41.8996) (width 0.2) (layer "F.Cu") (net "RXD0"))
 (segment (start 27.9502 37.6491) (end 27.9502 40.0294) (width 0.2) (layer "F.Cu") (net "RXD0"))
 (segment (start 31.8017 36.2217) (end 30.8151 37.2083) (width 0.2) (layer "F.Cu") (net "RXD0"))
 (segment (start 30.8151 37.2083) (end 28.391 37.2083) (width 0.2) (layer "F.Cu") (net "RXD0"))
 (segment (start 30.75 19.82) (end 31.8017 19.82) (width 0.2) (layer "F.Cu") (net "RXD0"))
 (segment (start 26.08 41.8996) (end 26.08 48.5) (width 0.2) (layer "F.Cu") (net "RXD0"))
 (segment (start 29.7233 30.9935) (end 29.4942 31.2226) (width 0.15) (layer "F.Cu") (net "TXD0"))
 (segment (start 29.7233 18.55) (end 29.7233 30.9935) (width 0.15) (layer "F.Cu") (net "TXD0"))
 (segment (start 30.75 18.55) (end 29.7233 18.55) (width 0.15) (layer "F.Cu") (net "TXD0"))
 (via (at 29.4942 31.2226) (size 0.6) (drill 0.3) (layers "F.Cu" "B.Cu") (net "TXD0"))
 (segment (start 29.4942 42.5458) (end 29.4942 31.2226) (width 0.2) (layer "B.Cu") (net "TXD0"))
 (segment (start 23.54 48.5) (end 29.4942 42.5458) (width 0.2) (layer "B.Cu") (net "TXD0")))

